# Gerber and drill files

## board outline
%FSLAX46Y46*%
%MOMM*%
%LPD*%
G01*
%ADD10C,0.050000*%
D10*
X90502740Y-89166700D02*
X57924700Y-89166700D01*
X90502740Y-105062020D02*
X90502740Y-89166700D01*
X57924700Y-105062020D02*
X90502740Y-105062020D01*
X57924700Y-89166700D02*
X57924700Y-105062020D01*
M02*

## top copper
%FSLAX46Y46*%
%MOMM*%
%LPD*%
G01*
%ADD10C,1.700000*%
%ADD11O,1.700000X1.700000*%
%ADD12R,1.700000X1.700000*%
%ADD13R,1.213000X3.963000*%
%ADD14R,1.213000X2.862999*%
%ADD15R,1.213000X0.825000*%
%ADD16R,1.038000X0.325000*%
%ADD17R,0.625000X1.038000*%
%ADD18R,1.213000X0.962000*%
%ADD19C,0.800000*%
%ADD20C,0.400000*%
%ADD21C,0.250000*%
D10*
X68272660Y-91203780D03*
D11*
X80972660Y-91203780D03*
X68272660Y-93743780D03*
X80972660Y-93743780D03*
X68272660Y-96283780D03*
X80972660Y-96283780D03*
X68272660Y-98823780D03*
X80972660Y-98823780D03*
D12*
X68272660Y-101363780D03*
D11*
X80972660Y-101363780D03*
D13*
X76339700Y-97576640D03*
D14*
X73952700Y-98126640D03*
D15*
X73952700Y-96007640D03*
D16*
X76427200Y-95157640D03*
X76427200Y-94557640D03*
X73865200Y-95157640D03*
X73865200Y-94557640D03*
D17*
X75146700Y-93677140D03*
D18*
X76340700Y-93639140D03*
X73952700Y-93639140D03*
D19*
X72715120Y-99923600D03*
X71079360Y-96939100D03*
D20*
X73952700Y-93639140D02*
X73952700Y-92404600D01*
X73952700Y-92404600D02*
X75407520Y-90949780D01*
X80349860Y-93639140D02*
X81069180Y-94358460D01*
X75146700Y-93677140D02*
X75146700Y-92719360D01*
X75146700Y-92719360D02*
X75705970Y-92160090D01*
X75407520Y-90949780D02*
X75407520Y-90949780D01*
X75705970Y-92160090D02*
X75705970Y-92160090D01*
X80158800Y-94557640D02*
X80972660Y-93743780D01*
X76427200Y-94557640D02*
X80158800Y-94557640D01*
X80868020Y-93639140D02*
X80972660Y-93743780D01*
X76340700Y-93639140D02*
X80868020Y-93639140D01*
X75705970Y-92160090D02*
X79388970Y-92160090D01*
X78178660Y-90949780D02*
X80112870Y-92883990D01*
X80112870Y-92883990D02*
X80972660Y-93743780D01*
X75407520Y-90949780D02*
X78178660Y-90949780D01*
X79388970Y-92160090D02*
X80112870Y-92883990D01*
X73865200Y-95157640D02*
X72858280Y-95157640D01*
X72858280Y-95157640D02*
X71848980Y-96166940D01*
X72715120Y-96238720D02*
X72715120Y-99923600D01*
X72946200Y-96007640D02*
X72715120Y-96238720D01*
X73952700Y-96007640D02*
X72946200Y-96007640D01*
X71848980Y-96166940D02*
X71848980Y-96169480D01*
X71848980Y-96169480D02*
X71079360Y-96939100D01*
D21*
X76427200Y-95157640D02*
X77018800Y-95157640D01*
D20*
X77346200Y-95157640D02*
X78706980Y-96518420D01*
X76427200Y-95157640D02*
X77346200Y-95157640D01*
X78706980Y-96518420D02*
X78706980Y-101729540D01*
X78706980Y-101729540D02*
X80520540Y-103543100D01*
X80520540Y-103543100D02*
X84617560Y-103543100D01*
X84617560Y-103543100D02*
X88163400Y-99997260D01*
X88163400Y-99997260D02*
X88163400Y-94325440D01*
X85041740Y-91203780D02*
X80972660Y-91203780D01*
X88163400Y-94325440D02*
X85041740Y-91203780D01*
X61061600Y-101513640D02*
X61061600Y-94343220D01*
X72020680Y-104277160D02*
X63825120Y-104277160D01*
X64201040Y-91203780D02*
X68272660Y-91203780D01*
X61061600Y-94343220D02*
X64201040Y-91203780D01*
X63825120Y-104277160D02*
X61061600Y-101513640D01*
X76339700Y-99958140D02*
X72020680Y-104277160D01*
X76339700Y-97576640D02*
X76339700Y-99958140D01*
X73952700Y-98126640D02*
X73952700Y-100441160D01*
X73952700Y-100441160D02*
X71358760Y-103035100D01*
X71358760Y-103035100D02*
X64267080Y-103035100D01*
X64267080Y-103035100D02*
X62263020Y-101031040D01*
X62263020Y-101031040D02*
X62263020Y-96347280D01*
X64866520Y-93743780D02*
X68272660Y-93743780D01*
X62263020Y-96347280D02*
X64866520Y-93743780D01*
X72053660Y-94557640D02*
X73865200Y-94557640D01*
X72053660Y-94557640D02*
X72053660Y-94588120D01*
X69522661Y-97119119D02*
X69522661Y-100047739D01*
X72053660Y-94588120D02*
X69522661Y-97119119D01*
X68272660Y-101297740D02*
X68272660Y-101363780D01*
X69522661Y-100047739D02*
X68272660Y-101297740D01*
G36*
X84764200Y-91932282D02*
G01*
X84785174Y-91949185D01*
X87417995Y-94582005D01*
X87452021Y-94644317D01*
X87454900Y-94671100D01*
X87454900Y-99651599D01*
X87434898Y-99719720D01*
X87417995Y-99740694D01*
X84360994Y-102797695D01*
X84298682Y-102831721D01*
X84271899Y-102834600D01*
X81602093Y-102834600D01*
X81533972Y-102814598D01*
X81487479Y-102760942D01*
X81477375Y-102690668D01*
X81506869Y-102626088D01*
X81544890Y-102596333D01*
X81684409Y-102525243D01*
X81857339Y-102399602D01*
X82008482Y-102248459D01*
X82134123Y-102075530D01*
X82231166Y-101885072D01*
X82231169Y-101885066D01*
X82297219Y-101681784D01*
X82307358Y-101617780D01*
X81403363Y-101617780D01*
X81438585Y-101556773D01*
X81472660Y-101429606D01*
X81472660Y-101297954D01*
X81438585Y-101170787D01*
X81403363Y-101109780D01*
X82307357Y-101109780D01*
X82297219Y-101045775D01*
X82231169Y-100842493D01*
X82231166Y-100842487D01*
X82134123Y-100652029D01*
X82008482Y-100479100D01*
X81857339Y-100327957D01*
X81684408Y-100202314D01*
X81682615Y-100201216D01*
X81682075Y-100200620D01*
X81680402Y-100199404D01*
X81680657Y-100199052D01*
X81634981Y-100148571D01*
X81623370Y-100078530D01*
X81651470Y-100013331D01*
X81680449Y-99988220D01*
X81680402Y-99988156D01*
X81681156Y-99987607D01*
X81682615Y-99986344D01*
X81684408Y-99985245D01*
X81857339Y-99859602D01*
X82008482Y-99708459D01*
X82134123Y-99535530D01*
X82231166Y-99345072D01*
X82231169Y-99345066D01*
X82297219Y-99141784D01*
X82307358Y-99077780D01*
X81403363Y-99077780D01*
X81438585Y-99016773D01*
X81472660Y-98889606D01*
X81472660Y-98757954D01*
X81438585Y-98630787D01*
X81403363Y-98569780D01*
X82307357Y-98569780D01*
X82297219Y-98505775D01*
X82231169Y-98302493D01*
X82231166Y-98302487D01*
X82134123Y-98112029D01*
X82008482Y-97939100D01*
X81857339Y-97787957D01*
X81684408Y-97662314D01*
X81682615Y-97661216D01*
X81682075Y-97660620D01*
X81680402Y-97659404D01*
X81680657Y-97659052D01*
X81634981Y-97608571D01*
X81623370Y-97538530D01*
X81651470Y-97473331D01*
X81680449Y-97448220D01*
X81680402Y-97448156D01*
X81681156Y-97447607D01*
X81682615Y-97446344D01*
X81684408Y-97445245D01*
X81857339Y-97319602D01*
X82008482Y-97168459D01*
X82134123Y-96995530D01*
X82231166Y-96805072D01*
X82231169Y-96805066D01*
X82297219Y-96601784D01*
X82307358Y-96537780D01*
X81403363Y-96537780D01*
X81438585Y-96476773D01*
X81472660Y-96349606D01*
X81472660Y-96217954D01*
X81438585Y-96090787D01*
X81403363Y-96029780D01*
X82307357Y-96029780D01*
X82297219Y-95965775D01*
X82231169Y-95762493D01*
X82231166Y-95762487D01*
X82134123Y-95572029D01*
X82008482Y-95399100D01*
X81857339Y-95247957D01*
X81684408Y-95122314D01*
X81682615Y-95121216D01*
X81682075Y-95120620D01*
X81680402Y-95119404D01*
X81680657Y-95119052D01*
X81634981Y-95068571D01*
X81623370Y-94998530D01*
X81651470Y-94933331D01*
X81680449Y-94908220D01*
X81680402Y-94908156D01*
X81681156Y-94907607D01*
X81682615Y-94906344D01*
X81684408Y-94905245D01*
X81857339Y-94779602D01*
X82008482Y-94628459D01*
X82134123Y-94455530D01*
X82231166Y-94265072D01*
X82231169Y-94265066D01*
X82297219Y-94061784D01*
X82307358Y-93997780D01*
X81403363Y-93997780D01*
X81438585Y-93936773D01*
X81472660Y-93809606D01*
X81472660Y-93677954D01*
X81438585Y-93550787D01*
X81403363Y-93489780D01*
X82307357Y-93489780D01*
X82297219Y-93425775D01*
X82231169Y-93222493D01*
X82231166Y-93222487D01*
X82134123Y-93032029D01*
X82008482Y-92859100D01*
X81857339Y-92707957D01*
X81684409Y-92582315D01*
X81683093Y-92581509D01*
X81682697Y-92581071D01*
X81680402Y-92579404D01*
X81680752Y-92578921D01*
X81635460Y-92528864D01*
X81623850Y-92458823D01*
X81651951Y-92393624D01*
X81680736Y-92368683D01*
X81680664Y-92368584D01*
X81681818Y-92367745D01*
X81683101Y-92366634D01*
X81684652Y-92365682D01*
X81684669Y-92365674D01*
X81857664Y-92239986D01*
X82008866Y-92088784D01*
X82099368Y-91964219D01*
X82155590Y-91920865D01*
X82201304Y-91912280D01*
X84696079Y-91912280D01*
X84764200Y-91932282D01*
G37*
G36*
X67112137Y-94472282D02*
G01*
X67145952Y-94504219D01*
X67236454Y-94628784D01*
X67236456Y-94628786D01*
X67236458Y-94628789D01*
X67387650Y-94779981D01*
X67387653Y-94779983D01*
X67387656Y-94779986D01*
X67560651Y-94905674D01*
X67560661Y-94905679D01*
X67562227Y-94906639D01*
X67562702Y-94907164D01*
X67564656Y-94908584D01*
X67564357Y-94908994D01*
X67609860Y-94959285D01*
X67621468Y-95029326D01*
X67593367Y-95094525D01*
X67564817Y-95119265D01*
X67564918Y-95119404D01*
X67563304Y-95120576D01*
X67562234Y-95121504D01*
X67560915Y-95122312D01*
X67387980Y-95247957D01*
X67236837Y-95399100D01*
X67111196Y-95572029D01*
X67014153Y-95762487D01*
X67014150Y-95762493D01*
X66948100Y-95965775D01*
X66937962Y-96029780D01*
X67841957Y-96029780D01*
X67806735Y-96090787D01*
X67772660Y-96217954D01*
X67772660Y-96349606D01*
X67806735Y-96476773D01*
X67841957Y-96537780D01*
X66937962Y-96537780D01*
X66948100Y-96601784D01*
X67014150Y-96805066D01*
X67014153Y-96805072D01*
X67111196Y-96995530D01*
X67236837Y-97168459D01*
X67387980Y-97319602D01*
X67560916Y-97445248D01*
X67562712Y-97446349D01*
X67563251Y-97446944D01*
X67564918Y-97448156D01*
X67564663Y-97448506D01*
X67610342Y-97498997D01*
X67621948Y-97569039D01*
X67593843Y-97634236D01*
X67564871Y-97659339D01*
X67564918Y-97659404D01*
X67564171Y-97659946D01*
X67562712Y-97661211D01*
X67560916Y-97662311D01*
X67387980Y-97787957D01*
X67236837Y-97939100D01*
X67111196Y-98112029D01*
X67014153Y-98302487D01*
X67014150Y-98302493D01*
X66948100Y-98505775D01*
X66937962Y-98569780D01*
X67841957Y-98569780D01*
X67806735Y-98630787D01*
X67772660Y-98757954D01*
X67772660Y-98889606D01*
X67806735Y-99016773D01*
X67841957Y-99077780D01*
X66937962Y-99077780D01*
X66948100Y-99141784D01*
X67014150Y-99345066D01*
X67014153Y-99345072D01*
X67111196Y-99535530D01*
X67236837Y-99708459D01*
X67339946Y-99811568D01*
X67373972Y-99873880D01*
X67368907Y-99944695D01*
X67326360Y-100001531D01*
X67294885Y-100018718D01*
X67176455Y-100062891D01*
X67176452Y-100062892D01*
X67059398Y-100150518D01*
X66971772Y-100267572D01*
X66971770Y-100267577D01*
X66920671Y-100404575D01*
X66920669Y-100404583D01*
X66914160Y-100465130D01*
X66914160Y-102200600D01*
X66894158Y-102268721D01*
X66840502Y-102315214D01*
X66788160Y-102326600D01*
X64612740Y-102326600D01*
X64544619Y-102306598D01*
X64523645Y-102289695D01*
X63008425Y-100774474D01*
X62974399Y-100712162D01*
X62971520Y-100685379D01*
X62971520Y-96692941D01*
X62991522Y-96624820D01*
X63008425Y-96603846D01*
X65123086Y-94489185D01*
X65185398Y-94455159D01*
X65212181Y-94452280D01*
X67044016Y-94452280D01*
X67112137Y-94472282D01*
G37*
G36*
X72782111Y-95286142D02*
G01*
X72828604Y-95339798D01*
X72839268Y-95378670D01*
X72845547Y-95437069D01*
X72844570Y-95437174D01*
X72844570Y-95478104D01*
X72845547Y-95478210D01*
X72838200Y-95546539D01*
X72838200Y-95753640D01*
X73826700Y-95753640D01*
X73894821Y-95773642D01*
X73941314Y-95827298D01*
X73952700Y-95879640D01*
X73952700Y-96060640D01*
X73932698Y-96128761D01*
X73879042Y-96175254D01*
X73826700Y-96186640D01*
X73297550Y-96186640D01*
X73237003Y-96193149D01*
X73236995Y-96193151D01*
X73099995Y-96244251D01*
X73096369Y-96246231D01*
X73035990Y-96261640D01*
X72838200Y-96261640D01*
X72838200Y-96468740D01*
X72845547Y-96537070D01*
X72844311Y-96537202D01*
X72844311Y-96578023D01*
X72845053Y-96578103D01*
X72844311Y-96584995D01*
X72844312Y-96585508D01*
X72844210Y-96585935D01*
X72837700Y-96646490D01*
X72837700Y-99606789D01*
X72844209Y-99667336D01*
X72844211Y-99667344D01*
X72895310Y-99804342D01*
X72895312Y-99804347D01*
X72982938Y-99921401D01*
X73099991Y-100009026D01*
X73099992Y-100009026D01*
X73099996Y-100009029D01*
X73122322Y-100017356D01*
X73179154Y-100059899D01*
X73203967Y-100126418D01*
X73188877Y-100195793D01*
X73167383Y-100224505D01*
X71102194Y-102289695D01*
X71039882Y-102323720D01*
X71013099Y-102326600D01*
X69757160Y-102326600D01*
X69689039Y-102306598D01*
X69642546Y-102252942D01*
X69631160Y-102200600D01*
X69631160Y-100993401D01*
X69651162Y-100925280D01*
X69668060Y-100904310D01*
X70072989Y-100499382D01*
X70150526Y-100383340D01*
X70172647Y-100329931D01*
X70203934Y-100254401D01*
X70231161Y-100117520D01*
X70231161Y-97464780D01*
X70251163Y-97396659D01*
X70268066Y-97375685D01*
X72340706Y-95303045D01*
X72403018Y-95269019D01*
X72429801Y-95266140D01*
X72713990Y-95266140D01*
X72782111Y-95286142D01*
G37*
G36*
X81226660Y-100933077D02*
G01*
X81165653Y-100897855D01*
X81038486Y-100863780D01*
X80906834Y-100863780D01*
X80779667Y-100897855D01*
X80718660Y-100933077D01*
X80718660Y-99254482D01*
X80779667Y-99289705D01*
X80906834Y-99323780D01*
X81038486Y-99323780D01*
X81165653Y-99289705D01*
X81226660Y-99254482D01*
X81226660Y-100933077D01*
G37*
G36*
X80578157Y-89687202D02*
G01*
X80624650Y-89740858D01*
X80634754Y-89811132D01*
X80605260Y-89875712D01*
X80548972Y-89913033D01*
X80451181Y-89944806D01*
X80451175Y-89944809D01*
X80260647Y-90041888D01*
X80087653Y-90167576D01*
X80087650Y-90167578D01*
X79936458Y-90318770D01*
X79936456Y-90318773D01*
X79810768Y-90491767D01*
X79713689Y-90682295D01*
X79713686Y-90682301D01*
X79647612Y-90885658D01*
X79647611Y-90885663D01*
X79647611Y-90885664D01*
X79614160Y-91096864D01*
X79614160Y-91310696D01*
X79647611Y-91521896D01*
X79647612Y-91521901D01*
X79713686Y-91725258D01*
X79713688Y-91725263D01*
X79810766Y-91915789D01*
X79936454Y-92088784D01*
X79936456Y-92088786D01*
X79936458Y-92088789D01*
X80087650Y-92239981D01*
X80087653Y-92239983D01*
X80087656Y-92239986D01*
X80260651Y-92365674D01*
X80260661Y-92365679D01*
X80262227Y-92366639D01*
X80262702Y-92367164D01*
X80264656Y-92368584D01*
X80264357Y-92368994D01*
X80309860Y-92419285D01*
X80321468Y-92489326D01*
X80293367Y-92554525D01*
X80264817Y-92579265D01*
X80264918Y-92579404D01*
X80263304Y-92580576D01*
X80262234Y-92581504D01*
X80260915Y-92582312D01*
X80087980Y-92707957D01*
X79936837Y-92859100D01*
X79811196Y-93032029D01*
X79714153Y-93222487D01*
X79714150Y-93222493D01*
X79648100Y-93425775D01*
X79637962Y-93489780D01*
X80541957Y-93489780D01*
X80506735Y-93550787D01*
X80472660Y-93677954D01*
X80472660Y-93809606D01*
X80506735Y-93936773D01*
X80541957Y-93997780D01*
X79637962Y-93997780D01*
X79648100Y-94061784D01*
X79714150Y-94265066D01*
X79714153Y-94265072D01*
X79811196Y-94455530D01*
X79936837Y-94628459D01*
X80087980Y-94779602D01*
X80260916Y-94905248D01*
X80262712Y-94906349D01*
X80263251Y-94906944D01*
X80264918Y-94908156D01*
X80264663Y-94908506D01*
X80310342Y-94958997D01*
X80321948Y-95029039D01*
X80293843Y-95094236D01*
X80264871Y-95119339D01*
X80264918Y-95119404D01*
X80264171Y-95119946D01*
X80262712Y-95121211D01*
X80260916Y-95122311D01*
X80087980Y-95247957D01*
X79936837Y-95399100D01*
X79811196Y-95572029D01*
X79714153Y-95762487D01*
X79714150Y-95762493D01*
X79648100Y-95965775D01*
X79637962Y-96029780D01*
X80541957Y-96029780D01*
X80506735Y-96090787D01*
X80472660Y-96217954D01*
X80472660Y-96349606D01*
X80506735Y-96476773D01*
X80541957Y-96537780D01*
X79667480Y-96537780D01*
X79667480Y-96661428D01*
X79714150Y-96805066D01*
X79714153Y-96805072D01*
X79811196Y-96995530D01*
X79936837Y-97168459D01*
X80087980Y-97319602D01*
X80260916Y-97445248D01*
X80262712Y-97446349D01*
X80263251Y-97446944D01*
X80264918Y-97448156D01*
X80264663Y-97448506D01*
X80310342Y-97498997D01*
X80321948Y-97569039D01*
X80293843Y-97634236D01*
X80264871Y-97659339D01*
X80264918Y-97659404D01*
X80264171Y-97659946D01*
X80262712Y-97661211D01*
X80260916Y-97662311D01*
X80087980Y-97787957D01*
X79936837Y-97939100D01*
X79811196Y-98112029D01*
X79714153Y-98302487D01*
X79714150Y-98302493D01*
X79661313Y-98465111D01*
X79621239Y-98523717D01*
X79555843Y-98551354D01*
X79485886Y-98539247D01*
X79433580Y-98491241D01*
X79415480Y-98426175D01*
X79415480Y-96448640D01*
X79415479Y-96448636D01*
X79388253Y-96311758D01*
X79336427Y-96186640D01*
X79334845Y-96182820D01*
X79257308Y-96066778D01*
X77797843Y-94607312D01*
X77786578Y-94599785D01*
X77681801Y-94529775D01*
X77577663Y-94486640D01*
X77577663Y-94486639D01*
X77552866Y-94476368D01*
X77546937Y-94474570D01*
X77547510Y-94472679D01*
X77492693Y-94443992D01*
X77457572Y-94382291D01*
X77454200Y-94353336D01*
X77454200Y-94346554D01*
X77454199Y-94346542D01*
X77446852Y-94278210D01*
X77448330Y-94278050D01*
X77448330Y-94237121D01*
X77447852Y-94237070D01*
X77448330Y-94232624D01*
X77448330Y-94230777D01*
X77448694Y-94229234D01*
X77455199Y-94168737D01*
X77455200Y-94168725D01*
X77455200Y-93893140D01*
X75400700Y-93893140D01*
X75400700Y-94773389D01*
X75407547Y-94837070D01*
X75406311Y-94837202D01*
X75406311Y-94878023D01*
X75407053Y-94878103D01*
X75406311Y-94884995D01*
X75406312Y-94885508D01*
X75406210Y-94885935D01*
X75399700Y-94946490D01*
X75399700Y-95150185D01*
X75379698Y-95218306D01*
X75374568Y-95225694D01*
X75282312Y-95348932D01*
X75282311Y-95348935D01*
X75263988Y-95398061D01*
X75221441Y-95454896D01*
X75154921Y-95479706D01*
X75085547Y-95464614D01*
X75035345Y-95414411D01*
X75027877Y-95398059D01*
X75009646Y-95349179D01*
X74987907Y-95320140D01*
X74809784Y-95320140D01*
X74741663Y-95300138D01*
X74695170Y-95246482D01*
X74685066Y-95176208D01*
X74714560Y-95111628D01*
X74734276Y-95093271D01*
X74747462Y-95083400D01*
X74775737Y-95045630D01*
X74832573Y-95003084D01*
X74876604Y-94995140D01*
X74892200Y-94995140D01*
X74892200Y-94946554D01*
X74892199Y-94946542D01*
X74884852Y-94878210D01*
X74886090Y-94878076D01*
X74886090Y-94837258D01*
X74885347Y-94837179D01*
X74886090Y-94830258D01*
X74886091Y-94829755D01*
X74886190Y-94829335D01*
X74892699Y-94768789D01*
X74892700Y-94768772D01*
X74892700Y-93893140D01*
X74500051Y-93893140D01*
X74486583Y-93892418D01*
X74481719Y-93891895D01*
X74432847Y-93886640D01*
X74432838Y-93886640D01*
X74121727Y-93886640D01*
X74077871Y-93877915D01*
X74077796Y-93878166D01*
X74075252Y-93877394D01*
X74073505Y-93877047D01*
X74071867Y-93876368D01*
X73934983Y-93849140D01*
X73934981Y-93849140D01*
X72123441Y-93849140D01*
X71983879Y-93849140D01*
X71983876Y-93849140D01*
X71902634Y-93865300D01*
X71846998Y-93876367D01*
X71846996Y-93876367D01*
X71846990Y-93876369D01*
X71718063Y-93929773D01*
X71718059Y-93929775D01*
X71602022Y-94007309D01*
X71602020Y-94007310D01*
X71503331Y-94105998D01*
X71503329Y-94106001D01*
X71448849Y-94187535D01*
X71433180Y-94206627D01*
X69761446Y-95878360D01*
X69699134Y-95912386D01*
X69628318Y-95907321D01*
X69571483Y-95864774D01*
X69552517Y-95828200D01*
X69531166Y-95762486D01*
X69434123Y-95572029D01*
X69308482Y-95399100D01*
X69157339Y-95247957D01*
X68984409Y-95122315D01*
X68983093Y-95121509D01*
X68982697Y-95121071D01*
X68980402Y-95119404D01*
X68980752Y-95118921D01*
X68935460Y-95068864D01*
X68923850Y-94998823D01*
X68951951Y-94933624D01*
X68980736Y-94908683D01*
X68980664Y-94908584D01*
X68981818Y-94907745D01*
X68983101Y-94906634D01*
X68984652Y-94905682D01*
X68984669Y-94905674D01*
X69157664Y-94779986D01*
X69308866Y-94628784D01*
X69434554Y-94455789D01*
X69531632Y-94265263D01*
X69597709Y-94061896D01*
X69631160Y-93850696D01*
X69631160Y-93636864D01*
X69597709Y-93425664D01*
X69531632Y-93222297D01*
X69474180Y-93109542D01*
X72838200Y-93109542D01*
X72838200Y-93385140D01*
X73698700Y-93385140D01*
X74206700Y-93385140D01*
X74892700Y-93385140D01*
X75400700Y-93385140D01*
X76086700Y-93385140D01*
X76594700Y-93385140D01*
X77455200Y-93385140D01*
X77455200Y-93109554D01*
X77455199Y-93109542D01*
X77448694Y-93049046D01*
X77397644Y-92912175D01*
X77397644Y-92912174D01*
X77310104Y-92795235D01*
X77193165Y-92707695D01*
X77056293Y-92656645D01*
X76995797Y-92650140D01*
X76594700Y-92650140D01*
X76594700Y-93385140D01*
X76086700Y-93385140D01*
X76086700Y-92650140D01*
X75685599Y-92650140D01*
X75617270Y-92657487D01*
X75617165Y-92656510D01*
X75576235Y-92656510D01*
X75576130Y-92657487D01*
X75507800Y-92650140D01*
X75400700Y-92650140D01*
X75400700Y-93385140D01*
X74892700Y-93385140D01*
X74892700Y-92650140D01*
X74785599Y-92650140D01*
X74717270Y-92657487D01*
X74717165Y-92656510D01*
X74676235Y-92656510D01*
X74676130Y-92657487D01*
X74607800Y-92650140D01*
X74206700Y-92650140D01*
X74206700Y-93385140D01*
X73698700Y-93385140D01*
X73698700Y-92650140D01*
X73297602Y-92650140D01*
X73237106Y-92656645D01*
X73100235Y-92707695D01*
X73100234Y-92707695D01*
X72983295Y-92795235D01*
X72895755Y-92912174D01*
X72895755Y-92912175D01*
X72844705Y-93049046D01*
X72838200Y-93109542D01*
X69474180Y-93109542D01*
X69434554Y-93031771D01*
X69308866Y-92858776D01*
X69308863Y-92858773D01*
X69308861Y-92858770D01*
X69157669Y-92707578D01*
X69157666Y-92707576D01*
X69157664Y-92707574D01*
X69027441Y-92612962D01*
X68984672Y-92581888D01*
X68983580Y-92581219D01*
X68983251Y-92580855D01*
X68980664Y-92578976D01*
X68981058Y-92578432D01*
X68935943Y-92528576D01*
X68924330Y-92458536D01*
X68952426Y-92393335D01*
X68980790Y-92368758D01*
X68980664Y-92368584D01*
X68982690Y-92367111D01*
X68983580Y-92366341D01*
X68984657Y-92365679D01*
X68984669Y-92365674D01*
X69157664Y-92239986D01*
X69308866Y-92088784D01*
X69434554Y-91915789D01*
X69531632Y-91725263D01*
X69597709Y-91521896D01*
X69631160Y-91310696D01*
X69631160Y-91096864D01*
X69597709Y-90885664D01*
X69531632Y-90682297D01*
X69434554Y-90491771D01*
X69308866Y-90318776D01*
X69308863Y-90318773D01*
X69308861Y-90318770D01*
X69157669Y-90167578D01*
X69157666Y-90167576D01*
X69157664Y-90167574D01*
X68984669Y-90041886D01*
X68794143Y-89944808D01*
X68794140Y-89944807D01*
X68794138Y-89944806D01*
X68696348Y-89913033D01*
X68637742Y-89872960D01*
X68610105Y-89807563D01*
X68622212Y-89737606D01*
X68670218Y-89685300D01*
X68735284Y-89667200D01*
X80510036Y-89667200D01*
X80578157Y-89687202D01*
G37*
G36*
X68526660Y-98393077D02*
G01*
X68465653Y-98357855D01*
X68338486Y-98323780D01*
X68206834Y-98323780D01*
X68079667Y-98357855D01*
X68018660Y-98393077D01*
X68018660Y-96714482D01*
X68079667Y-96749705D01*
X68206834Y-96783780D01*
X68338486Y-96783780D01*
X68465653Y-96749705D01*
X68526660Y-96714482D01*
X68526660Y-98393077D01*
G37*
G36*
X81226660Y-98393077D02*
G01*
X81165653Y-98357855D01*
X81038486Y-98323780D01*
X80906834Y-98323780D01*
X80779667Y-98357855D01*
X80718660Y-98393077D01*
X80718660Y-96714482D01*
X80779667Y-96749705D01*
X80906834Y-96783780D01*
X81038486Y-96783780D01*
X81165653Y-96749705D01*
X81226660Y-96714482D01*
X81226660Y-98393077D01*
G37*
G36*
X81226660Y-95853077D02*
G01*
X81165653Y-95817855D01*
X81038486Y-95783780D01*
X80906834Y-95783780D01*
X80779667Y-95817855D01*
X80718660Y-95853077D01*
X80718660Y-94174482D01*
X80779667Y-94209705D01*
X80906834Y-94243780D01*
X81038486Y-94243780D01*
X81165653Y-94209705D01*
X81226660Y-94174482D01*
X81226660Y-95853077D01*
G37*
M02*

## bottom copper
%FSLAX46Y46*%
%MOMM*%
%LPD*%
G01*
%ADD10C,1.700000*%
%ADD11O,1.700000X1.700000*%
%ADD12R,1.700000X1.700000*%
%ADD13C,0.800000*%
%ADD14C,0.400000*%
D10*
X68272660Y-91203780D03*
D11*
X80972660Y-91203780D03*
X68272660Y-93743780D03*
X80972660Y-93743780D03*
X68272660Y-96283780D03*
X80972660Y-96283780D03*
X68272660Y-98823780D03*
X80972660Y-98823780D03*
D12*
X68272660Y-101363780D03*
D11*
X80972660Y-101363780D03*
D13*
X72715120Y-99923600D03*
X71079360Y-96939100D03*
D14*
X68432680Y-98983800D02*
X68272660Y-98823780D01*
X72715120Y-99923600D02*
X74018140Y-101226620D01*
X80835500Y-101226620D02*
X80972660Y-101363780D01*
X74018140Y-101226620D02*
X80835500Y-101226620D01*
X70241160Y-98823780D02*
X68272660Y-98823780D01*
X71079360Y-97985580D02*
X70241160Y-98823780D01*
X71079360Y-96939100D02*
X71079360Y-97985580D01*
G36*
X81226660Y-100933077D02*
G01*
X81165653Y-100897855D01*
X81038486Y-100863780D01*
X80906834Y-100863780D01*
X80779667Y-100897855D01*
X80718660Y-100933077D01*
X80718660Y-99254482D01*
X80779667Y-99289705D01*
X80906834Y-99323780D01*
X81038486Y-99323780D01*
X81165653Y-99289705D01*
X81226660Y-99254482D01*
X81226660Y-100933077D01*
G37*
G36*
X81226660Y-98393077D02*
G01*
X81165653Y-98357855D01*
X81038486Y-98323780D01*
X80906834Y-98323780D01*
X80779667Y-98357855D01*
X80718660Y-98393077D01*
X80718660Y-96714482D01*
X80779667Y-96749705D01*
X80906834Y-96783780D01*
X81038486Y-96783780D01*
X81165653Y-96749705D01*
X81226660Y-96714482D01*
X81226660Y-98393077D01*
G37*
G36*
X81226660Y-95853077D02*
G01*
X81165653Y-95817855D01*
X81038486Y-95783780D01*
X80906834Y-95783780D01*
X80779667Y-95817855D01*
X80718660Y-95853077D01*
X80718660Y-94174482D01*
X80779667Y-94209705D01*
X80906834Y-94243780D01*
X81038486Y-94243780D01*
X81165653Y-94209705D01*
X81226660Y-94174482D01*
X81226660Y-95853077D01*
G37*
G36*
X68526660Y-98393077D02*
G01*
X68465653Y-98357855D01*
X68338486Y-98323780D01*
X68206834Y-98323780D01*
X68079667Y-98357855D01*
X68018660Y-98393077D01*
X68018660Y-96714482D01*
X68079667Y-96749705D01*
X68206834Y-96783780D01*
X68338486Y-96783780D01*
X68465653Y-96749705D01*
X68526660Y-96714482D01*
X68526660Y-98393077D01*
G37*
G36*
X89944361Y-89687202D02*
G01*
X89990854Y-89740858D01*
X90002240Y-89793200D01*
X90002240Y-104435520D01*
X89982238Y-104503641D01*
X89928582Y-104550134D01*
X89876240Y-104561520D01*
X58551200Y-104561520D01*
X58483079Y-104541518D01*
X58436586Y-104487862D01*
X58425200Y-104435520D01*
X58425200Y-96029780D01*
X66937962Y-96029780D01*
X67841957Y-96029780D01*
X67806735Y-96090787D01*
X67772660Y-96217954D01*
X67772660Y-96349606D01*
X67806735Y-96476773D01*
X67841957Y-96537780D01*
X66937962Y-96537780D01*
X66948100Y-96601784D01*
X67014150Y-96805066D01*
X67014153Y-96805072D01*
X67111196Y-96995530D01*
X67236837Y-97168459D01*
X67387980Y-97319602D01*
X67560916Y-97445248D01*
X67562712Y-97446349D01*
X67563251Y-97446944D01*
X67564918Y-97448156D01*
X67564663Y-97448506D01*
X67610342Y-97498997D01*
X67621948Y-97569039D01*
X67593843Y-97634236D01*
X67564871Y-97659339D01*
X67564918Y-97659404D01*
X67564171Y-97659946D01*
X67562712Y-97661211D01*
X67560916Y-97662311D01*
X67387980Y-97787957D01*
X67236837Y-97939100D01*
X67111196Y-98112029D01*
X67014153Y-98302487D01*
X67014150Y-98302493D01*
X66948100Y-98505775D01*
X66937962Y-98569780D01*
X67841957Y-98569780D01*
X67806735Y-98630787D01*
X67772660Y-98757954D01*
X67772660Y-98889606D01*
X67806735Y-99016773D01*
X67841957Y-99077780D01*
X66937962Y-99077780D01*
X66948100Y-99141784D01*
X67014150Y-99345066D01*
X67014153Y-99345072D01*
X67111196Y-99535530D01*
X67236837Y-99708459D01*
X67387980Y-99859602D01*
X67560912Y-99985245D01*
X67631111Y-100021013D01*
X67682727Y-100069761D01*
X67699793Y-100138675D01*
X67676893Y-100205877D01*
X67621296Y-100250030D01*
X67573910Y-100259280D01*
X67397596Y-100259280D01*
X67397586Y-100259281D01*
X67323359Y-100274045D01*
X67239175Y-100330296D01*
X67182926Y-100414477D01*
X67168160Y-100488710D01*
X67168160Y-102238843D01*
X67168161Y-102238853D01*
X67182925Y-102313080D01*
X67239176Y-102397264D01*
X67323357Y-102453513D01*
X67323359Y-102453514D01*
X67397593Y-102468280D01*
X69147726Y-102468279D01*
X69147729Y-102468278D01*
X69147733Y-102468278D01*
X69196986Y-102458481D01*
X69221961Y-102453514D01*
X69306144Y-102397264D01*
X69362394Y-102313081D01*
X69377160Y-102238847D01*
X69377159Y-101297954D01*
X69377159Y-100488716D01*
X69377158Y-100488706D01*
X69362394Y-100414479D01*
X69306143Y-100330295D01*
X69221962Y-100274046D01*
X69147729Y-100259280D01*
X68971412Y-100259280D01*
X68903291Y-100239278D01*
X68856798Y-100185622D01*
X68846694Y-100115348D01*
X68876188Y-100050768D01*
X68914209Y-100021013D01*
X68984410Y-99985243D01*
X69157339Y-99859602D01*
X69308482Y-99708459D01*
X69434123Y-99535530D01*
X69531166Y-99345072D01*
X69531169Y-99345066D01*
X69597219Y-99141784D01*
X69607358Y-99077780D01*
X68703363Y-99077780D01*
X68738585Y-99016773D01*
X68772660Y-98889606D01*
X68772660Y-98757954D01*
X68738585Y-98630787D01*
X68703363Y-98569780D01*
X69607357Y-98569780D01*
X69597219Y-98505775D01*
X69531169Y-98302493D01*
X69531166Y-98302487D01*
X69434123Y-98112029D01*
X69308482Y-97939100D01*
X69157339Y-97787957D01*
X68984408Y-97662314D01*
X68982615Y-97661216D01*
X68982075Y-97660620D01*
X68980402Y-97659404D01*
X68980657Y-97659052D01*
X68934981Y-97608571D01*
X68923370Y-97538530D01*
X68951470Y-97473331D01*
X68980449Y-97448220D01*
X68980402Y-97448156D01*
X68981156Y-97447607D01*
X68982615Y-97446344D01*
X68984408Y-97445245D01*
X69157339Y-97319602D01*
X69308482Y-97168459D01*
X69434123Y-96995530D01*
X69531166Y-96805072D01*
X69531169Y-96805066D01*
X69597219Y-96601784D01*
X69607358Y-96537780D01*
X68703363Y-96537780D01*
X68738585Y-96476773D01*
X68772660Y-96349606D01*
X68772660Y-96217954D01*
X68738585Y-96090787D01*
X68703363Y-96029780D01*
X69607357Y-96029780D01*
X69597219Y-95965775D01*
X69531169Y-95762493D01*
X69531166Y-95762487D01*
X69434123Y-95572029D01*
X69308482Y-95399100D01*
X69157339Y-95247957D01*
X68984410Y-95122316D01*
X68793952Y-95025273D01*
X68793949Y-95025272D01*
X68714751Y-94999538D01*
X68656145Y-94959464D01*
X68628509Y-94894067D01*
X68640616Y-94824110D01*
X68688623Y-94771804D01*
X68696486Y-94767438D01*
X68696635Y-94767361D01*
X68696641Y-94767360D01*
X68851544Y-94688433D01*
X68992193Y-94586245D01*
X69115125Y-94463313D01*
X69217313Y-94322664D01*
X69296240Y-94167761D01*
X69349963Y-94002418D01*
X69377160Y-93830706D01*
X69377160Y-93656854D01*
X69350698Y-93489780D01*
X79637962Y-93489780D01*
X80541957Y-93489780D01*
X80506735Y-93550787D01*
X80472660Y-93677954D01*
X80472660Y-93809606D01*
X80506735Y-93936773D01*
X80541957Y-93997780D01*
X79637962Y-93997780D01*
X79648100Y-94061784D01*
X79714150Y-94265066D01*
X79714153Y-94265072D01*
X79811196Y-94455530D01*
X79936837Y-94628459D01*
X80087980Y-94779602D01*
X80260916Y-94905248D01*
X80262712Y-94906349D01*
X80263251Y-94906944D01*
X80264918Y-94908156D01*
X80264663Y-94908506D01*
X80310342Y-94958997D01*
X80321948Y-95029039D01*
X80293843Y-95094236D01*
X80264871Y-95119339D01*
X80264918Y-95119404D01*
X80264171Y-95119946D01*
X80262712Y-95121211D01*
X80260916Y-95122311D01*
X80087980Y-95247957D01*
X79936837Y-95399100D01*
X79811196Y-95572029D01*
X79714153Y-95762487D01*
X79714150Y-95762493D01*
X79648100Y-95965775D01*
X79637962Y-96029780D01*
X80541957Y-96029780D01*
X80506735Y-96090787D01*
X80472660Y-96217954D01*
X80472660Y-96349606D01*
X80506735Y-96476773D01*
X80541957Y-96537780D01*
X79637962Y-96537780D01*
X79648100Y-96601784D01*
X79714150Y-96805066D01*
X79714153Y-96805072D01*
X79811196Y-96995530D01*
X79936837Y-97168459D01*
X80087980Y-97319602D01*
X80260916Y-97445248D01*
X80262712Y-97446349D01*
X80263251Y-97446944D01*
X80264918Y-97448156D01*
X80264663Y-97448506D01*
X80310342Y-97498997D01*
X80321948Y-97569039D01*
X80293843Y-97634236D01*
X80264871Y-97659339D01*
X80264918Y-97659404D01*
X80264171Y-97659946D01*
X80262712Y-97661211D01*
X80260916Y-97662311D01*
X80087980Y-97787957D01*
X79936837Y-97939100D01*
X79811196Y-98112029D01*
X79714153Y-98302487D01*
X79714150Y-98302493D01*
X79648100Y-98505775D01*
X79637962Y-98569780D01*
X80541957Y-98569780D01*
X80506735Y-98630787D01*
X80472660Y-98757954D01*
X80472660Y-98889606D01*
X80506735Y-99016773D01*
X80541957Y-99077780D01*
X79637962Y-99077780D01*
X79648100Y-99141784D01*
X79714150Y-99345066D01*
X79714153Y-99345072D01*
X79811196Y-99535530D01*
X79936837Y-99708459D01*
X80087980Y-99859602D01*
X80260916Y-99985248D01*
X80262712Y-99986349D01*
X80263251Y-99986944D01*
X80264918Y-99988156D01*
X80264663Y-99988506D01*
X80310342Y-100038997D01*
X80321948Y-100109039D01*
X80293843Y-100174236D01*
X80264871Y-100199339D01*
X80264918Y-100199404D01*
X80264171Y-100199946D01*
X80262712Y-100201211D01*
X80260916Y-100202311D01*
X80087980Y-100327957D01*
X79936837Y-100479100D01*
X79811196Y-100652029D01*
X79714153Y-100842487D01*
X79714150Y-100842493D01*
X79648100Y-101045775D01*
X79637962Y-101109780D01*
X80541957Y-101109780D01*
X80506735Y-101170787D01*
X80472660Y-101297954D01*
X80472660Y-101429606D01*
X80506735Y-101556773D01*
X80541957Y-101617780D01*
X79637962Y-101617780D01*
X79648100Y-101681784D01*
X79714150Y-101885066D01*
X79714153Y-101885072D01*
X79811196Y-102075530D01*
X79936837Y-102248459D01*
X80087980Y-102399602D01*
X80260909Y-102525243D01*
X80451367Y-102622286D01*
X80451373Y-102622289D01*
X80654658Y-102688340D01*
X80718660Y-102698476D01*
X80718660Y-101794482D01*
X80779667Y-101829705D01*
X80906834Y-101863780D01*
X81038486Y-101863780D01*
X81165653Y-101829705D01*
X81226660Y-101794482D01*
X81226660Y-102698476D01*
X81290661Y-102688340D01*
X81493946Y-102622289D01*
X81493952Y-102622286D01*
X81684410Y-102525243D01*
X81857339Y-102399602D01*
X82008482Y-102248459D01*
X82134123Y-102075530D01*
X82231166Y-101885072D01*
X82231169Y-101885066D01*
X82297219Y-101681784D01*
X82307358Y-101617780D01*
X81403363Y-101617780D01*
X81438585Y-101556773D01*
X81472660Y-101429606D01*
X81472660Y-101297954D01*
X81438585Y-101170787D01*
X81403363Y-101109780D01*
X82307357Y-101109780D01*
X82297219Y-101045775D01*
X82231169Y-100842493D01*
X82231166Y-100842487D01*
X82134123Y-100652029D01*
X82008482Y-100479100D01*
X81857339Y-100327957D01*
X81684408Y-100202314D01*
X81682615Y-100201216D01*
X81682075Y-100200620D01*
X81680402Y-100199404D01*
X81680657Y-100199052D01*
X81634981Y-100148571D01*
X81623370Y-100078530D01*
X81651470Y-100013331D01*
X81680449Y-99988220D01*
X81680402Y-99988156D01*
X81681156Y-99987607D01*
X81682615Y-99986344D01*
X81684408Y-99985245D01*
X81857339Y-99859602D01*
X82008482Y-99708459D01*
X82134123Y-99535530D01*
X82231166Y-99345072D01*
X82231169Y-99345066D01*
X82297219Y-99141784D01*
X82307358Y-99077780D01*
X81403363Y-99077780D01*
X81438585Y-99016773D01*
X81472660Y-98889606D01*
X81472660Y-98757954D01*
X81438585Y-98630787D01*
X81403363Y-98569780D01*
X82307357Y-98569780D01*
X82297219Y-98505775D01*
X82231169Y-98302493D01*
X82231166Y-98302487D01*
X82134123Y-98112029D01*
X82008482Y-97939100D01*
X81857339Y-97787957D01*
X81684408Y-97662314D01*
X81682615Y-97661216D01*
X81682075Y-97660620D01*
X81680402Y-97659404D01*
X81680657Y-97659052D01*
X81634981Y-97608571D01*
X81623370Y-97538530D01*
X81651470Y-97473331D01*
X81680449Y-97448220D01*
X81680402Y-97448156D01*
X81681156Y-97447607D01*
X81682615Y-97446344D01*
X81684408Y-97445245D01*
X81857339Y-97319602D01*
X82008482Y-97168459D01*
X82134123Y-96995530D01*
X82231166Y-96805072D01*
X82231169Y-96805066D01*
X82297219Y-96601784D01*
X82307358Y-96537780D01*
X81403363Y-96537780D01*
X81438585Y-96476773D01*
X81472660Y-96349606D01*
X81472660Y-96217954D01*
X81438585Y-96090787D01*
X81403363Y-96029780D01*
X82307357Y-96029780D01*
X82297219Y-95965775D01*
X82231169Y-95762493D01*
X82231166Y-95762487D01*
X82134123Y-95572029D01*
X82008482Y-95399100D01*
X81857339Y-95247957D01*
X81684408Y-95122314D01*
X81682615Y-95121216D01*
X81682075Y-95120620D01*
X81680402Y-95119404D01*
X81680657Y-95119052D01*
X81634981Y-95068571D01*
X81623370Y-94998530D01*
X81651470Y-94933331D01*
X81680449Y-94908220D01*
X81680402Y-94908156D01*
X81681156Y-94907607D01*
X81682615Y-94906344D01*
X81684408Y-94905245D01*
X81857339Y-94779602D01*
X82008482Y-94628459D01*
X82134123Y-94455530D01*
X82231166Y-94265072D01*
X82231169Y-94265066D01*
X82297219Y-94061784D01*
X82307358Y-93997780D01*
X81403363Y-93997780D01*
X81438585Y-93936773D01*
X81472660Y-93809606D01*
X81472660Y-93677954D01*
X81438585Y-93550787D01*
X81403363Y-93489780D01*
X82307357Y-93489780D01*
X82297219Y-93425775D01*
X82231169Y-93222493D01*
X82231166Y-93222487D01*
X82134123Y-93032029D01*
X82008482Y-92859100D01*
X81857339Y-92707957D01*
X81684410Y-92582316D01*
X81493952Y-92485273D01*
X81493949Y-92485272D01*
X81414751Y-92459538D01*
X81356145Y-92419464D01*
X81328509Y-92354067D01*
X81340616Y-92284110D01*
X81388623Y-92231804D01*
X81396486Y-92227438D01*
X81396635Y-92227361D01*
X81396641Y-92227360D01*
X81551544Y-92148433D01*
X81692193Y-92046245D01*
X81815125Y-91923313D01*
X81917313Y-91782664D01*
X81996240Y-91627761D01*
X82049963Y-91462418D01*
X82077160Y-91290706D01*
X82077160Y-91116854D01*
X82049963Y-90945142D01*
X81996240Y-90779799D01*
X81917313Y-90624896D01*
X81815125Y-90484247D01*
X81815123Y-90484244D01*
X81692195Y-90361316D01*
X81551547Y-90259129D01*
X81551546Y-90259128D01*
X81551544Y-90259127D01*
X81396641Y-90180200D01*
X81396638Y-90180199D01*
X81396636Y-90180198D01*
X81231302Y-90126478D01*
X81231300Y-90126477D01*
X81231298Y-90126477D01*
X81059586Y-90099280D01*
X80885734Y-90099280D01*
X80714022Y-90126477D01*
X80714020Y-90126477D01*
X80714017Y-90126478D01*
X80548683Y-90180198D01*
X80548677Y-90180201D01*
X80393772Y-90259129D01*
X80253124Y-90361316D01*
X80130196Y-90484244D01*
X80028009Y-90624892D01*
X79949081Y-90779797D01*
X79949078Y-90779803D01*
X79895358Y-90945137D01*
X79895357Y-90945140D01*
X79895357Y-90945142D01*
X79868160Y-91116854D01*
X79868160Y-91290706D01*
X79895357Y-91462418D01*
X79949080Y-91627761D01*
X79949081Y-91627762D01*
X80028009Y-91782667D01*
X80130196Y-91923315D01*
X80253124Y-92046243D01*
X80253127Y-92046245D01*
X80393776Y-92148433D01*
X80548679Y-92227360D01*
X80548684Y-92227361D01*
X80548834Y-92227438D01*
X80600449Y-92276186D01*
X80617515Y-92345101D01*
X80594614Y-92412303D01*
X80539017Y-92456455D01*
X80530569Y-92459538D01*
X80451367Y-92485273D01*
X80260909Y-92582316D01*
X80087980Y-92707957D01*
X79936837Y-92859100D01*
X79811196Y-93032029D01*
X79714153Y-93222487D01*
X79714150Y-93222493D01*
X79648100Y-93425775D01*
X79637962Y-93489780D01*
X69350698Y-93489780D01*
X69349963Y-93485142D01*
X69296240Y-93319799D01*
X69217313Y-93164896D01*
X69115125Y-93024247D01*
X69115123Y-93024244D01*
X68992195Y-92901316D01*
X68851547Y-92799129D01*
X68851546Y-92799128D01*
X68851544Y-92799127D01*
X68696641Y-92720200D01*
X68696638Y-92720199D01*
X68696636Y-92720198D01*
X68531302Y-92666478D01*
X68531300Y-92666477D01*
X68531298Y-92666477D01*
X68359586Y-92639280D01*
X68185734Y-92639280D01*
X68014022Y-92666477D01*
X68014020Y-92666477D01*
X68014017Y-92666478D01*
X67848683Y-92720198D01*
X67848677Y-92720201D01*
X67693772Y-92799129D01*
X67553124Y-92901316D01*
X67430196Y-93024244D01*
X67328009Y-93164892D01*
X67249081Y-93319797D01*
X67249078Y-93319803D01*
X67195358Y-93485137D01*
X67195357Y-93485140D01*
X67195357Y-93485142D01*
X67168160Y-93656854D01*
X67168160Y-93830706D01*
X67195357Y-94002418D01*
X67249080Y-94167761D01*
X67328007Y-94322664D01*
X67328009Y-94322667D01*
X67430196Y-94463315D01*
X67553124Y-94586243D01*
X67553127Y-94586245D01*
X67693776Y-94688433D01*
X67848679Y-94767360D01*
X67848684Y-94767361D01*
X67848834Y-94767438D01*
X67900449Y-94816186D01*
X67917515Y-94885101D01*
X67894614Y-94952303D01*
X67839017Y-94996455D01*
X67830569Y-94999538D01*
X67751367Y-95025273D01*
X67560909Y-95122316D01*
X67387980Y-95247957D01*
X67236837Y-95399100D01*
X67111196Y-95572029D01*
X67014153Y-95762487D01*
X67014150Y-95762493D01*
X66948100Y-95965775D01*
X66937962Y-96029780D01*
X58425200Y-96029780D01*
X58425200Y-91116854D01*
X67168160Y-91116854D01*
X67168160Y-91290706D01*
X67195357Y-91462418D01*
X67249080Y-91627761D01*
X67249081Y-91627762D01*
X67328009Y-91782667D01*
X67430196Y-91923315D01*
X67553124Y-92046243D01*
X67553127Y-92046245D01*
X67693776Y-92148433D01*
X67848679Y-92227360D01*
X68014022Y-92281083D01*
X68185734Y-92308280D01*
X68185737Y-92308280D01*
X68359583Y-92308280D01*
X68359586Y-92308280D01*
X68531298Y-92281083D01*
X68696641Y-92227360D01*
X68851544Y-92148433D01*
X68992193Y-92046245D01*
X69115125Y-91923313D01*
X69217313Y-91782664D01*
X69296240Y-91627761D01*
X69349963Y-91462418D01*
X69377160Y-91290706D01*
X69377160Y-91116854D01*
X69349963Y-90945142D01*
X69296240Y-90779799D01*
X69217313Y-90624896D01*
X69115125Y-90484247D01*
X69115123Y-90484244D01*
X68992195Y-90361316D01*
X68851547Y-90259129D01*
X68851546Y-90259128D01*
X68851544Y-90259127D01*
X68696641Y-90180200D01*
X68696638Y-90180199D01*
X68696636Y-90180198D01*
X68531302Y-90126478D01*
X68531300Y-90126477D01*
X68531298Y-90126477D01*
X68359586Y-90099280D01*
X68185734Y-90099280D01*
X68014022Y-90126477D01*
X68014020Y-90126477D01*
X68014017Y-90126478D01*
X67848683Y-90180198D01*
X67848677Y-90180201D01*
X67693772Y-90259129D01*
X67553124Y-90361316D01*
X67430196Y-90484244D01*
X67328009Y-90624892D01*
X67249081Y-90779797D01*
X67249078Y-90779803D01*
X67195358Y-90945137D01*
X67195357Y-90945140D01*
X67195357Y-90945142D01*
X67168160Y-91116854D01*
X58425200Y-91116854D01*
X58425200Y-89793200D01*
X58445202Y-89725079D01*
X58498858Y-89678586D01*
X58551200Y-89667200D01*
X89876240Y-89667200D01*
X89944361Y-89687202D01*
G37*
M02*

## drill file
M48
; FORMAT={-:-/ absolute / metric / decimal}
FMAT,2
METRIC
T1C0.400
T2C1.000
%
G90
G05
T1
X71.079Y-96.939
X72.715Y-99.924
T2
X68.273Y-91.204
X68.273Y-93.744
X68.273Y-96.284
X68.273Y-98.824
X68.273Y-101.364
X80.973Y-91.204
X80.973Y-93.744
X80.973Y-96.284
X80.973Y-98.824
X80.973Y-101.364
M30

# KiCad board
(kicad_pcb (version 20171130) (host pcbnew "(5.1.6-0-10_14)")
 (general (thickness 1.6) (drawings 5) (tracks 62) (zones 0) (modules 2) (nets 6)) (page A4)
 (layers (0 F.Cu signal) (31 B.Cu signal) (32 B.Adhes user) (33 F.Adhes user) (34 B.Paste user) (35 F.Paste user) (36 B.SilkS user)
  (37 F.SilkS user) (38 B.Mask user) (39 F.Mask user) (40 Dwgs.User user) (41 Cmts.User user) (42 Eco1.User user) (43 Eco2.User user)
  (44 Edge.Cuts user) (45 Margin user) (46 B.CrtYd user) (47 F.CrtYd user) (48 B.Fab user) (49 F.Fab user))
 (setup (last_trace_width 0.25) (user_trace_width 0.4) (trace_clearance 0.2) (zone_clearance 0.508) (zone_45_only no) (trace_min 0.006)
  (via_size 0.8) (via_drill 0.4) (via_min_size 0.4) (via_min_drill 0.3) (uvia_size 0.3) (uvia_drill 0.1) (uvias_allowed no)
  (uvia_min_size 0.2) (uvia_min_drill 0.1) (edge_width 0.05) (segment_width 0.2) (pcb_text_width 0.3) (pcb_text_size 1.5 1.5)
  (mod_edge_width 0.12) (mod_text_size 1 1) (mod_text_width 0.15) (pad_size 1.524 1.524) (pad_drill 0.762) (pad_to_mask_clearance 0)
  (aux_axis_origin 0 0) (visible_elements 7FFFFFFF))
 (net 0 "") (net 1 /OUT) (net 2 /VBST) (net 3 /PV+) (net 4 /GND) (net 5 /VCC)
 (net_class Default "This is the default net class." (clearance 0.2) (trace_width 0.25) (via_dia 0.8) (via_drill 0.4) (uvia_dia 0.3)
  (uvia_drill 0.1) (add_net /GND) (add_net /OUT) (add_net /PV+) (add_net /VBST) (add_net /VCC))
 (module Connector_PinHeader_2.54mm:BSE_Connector (layer F.Cu) (at 68.27266 91.20378)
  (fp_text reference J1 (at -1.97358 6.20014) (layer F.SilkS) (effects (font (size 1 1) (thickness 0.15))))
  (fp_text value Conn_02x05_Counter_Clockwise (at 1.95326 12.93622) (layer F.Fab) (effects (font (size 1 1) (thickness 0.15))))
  (pad 5 thru_hole circle (at 0 0) (size 1.7 1.7) (drill 1) (layers *.Cu *.Mask) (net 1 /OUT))
  (pad 6 thru_hole oval (at 12.7 0) (size 1.7 1.7) (drill 1) (layers *.Cu *.Mask) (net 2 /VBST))
  (pad 4 thru_hole oval (at 0 2.54) (size 1.7 1.7) (drill 1) (layers *.Cu *.Mask) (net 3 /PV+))
  (pad 7 thru_hole oval (at 12.7 2.54) (size 1.7 1.7) (drill 1) (layers *.Cu *.Mask) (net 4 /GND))
  (pad 3 thru_hole oval (at 0 5.08) (size 1.7 1.7) (drill 1) (layers *.Cu *.Mask) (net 4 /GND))
  (pad 8 thru_hole oval (at 12.7 5.08) (size 1.7 1.7) (drill 1) (layers *.Cu *.Mask) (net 4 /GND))
  (pad 2 thru_hole oval (at 0 7.62) (size 1.7 1.7) (drill 1) (layers *.Cu *.Mask) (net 4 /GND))
  (pad 9 thru_hole oval (at 12.7 7.62) (size 1.7 1.7) (drill 1) (layers *.Cu *.Mask) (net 4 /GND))
  (pad 1 thru_hole rect (at 0 10.16) (size 1.7 1.7) (drill 1) (layers *.Cu *.Mask) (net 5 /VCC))
  (pad 10 thru_hole oval (at 12.7 10.16) (size 1.7 1.7) (drill 1) (layers *.Cu *.Mask) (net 4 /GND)))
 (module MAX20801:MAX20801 (layer F.Cu) (at 78.4262 94.42814)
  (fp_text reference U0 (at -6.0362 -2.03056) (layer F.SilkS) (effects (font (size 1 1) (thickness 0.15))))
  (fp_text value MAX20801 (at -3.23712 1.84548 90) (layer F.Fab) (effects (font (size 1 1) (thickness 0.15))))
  (pad 5 smd rect (at -2.0865 3.1485) (size 1.213 3.963) (layers F.Cu F.Paste F.Mask) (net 1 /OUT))
  (pad 4 smd rect (at -4.4735 3.6985) (size 1.213 2.862999) (layers F.Cu F.Paste F.Mask) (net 3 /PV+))
  (pad 3 smd rect (at -4.4735 1.5795) (size 1.213 0.825) (layers F.Cu F.Paste F.Mask) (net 4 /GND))
  (pad 6 smd rect (at -1.999 0.7295) (size 1.038 0.325) (layers F.Cu F.Paste F.Mask) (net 2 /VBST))
  (pad 7 smd rect (at -1.999 0.1295) (size 1.038 0.325) (layers F.Cu F.Paste F.Mask) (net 4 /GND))
  (pad 2 smd rect (at -4.561 0.7295) (size 1.038 0.325) (layers F.Cu F.Paste F.Mask) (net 4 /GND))
  (pad 1 smd rect (at -4.561 0.1295) (size 1.038 0.325) (layers F.Cu F.Paste F.Mask) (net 5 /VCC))
  (pad 9 smd rect (at -3.2795 -0.751) (size 0.625 1.038) (layers F.Cu F.Paste F.Mask) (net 4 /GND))
  (pad 8 smd rect (at -2.0855 -0.789) (size 1.213 0.962) (layers F.Cu F.Paste F.Mask) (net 4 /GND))
  (pad 10 smd rect (at -4.4735 -0.789) (size 1.213 0.962) (layers F.Cu F.Paste F.Mask) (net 4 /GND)))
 (gr_line (start 90.50274 89.1667) (end 57.9247 89.1667) (layer Edge.Cuts) (width 0.05))
 (gr_line (start 90.50274 105.06202) (end 90.50274 89.1667) (layer Edge.Cuts) (width 0.05))
 (gr_line (start 57.9247 105.06202) (end 90.50274 105.06202) (layer Edge.Cuts) (width 0.05))
 (gr_line (start 57.9247 89.1667) (end 57.9247 105.06202) (layer Edge.Cuts) (width 0.05))
 (segment (start 73.9527 93.63914) (end 73.9527 92.4046) (width 0.4) (layer F.Cu) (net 4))
 (segment (start 73.9527 92.4046) (end 75.40752 90.94978) (width 0.4) (layer F.Cu) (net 4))
 (segment (start 80.34986 93.63914) (end 81.06918 94.35846) (width 0.4) (layer F.Cu) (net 4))
 (segment (start 75.1467 93.67714) (end 75.1467 92.71936) (width 0.4) (layer F.Cu) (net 4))
 (segment (start 75.1467 92.71936) (end 75.70597 92.16009) (width 0.4) (layer F.Cu) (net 4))
 (segment (start 75.40752 90.94978) (end 75.40752 90.94978) (width 0.4) (layer F.Cu) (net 4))
 (segment (start 75.70597 92.16009) (end 75.70597 92.16009) (width 0.4) (layer F.Cu) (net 4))
 (segment (start 80.1588 94.55764) (end 80.97266 93.74378) (width 0.4) (layer F.Cu) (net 4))
 (segment (start 76.4272 94.55764) (end 80.1588 94.55764) (width 0.4) (layer F.Cu) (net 4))
 (segment (start 80.86802 93.63914) (end 80.97266 93.74378) (width 0.4) (layer F.Cu) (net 4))
 (segment (start 76.3407 93.63914) (end 80.86802 93.63914) (width 0.4) (layer F.Cu) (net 4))
 (segment (start 75.70597 92.16009) (end 79.38897 92.16009) (width 0.4) (layer F.Cu) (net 4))
 (segment (start 78.17866 90.94978) (end 80.11287 92.88399) (width 0.4) (layer F.Cu) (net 4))
 (segment (start 80.11287 92.88399) (end 80.97266 93.74378) (width 0.4) (layer F.Cu) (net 4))
 (segment (start 75.40752 90.94978) (end 78.17866 90.94978) (width 0.4) (layer F.Cu) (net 4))
 (segment (start 79.38897 92.16009) (end 80.11287 92.88399) (width 0.4) (layer F.Cu) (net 4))
 (segment (start 73.8652 95.15764) (end 72.85828 95.15764) (width 0.4) (layer F.Cu) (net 4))
 (segment (start 72.85828 95.15764) (end 71.84898 96.16694) (width 0.4) (layer F.Cu) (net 4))
 (segment (start 68.43268 98.9838) (end 68.27266 98.82378) (width 0.4) (layer B.Cu) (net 4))
 (via (at 72.71512 99.9236) (size 0.8) (drill 0.4) (layers F.Cu B.Cu) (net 4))
 (segment (start 72.71512 96.23872) (end 72.71512 99.9236) (width 0.4) (layer F.Cu) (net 4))
 (segment (start 72.9462 96.00764) (end 72.71512 96.23872) (width 0.4) (layer F.Cu) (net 4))
 (segment (start 73.9527 96.00764) (end 72.9462 96.00764) (width 0.4) (layer F.Cu) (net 4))
 (segment (start 72.71512 99.9236) (end 74.01814 101.22662) (width 0.4) (layer B.Cu) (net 4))
 (segment (start 80.8355 101.22662) (end 80.97266 101.36378) (width 0.4) (layer B.Cu) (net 4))
 (segment (start 74.01814 101.22662) (end 80.8355 101.22662) (width 0.4) (layer B.Cu) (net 4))
 (segment (start 71.84898 96.16694) (end 71.84898 96.16948) (width 0.4) (layer F.Cu) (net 4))
 (via (at 71.07936 96.9391) (size 0.8) (drill 0.4) (layers F.Cu B.Cu) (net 4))
 (segment (start 71.84898 96.16948) (end 71.07936 96.9391) (width 0.4) (layer F.Cu) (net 4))
 (segment (start 70.24116 98.82378) (end 68.27266 98.82378) (width 0.4) (layer B.Cu) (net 4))
 (segment (start 71.07936 97.98558) (end 70.24116 98.82378) (width 0.4) (layer B.Cu) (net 4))
 (segment (start 71.07936 96.9391) (end 71.07936 97.98558) (width 0.4) (layer B.Cu) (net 4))
 (segment (start 76.4272 95.15764) (end 77.0188 95.15764) (width 0.25) (layer F.Cu) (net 2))
 (segment (start 77.3462 95.15764) (end 78.70698 96.51842) (width 0.4) (layer F.Cu) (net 2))
 (segment (start 76.4272 95.15764) (end 77.3462 95.15764) (width 0.4) (layer F.Cu) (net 2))
 (segment (start 78.70698 96.51842) (end 78.70698 101.72954) (width 0.4) (layer F.Cu) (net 2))
 (segment (start 78.70698 101.72954) (end 80.52054 103.5431) (width 0.4) (layer F.Cu) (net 2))
 (segment (start 80.52054 103.5431) (end 84.61756 103.5431) (width 0.4) (layer F.Cu) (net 2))
 (segment (start 84.61756 103.5431) (end 88.1634 99.99726) (width 0.4) (layer F.Cu) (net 2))
 (segment (start 88.1634 99.99726) (end 88.1634 94.32544) (width 0.4) (layer F.Cu) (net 2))
 (segment (start 85.04174 91.20378) (end 80.97266 91.20378) (width 0.4) (layer F.Cu) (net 2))
 (segment (start 88.1634 94.32544) (end 85.04174 91.20378) (width 0.4) (layer F.Cu) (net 2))
 (segment (start 61.0616 101.51364) (end 61.0616 94.34322) (width 0.4) (layer F.Cu) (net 1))
 (segment (start 72.02068 104.27716) (end 63.82512 104.27716) (width 0.4) (layer F.Cu) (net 1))
 (segment (start 64.20104 91.20378) (end 68.27266 91.20378) (width 0.4) (layer F.Cu) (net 1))
 (segment (start 61.0616 94.34322) (end 64.20104 91.20378) (width 0.4) (layer F.Cu) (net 1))
 (segment (start 63.82512 104.27716) (end 61.0616 101.51364) (width 0.4) (layer F.Cu) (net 1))
 (segment (start 76.3397 99.95814) (end 72.02068 104.27716) (width 0.4) (layer F.Cu) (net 1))
 (segment (start 76.3397 97.57664) (end 76.3397 99.95814) (width 0.4) (layer F.Cu) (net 1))
 (segment (start 73.9527 98.12664) (end 73.9527 100.44116) (width 0.4) (layer F.Cu) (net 3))
 (segment (start 73.9527 100.44116) (end 71.35876 103.0351) (width 0.4) (layer F.Cu) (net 3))
 (segment (start 71.35876 103.0351) (end 64.26708 103.0351) (width 0.4) (layer F.Cu) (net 3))
 (segment (start 64.26708 103.0351) (end 62.26302 101.03104) (width 0.4) (layer F.Cu) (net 3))
 (segment (start 62.26302 101.03104) (end 62.26302 96.34728) (width 0.4) (layer F.Cu) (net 3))
 (segment (start 64.86652 93.74378) (end 68.27266 93.74378) (width 0.4) (layer F.Cu) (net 3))
 (segment (start 62.26302 96.34728) (end 64.86652 93.74378) (width 0.4) (layer F.Cu) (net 3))
 (segment (start 72.05366 94.55764) (end 73.8652 94.55764) (width 0.4) (layer F.Cu) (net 5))
 (segment (start 72.05366 94.55764) (end 72.05366 94.58812) (width 0.4) (layer F.Cu) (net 5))
 (segment (start 69.522661 97.119119) (end 69.522661 100.047739) (width 0.4) (layer F.Cu) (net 5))
 (segment (start 72.05366 94.58812) (end 69.522661 97.119119) (width 0.4) (layer F.Cu) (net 5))
 (segment (start 68.27266 101.29774) (end 68.27266 101.36378) (width 0.4) (layer F.Cu) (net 5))
 (segment (start 69.522661 100.047739) (end 68.27266 101.29774) (width 0.4) (layer F.Cu) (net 5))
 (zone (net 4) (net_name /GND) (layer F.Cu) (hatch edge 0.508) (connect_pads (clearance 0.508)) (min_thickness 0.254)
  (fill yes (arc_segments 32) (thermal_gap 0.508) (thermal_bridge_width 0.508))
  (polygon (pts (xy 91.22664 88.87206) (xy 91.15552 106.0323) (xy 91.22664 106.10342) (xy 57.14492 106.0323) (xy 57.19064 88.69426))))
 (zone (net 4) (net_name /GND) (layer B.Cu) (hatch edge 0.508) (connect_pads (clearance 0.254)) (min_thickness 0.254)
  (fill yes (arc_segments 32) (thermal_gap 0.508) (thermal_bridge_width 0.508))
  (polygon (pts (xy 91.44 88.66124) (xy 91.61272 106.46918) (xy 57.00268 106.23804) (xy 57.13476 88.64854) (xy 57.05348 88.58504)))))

